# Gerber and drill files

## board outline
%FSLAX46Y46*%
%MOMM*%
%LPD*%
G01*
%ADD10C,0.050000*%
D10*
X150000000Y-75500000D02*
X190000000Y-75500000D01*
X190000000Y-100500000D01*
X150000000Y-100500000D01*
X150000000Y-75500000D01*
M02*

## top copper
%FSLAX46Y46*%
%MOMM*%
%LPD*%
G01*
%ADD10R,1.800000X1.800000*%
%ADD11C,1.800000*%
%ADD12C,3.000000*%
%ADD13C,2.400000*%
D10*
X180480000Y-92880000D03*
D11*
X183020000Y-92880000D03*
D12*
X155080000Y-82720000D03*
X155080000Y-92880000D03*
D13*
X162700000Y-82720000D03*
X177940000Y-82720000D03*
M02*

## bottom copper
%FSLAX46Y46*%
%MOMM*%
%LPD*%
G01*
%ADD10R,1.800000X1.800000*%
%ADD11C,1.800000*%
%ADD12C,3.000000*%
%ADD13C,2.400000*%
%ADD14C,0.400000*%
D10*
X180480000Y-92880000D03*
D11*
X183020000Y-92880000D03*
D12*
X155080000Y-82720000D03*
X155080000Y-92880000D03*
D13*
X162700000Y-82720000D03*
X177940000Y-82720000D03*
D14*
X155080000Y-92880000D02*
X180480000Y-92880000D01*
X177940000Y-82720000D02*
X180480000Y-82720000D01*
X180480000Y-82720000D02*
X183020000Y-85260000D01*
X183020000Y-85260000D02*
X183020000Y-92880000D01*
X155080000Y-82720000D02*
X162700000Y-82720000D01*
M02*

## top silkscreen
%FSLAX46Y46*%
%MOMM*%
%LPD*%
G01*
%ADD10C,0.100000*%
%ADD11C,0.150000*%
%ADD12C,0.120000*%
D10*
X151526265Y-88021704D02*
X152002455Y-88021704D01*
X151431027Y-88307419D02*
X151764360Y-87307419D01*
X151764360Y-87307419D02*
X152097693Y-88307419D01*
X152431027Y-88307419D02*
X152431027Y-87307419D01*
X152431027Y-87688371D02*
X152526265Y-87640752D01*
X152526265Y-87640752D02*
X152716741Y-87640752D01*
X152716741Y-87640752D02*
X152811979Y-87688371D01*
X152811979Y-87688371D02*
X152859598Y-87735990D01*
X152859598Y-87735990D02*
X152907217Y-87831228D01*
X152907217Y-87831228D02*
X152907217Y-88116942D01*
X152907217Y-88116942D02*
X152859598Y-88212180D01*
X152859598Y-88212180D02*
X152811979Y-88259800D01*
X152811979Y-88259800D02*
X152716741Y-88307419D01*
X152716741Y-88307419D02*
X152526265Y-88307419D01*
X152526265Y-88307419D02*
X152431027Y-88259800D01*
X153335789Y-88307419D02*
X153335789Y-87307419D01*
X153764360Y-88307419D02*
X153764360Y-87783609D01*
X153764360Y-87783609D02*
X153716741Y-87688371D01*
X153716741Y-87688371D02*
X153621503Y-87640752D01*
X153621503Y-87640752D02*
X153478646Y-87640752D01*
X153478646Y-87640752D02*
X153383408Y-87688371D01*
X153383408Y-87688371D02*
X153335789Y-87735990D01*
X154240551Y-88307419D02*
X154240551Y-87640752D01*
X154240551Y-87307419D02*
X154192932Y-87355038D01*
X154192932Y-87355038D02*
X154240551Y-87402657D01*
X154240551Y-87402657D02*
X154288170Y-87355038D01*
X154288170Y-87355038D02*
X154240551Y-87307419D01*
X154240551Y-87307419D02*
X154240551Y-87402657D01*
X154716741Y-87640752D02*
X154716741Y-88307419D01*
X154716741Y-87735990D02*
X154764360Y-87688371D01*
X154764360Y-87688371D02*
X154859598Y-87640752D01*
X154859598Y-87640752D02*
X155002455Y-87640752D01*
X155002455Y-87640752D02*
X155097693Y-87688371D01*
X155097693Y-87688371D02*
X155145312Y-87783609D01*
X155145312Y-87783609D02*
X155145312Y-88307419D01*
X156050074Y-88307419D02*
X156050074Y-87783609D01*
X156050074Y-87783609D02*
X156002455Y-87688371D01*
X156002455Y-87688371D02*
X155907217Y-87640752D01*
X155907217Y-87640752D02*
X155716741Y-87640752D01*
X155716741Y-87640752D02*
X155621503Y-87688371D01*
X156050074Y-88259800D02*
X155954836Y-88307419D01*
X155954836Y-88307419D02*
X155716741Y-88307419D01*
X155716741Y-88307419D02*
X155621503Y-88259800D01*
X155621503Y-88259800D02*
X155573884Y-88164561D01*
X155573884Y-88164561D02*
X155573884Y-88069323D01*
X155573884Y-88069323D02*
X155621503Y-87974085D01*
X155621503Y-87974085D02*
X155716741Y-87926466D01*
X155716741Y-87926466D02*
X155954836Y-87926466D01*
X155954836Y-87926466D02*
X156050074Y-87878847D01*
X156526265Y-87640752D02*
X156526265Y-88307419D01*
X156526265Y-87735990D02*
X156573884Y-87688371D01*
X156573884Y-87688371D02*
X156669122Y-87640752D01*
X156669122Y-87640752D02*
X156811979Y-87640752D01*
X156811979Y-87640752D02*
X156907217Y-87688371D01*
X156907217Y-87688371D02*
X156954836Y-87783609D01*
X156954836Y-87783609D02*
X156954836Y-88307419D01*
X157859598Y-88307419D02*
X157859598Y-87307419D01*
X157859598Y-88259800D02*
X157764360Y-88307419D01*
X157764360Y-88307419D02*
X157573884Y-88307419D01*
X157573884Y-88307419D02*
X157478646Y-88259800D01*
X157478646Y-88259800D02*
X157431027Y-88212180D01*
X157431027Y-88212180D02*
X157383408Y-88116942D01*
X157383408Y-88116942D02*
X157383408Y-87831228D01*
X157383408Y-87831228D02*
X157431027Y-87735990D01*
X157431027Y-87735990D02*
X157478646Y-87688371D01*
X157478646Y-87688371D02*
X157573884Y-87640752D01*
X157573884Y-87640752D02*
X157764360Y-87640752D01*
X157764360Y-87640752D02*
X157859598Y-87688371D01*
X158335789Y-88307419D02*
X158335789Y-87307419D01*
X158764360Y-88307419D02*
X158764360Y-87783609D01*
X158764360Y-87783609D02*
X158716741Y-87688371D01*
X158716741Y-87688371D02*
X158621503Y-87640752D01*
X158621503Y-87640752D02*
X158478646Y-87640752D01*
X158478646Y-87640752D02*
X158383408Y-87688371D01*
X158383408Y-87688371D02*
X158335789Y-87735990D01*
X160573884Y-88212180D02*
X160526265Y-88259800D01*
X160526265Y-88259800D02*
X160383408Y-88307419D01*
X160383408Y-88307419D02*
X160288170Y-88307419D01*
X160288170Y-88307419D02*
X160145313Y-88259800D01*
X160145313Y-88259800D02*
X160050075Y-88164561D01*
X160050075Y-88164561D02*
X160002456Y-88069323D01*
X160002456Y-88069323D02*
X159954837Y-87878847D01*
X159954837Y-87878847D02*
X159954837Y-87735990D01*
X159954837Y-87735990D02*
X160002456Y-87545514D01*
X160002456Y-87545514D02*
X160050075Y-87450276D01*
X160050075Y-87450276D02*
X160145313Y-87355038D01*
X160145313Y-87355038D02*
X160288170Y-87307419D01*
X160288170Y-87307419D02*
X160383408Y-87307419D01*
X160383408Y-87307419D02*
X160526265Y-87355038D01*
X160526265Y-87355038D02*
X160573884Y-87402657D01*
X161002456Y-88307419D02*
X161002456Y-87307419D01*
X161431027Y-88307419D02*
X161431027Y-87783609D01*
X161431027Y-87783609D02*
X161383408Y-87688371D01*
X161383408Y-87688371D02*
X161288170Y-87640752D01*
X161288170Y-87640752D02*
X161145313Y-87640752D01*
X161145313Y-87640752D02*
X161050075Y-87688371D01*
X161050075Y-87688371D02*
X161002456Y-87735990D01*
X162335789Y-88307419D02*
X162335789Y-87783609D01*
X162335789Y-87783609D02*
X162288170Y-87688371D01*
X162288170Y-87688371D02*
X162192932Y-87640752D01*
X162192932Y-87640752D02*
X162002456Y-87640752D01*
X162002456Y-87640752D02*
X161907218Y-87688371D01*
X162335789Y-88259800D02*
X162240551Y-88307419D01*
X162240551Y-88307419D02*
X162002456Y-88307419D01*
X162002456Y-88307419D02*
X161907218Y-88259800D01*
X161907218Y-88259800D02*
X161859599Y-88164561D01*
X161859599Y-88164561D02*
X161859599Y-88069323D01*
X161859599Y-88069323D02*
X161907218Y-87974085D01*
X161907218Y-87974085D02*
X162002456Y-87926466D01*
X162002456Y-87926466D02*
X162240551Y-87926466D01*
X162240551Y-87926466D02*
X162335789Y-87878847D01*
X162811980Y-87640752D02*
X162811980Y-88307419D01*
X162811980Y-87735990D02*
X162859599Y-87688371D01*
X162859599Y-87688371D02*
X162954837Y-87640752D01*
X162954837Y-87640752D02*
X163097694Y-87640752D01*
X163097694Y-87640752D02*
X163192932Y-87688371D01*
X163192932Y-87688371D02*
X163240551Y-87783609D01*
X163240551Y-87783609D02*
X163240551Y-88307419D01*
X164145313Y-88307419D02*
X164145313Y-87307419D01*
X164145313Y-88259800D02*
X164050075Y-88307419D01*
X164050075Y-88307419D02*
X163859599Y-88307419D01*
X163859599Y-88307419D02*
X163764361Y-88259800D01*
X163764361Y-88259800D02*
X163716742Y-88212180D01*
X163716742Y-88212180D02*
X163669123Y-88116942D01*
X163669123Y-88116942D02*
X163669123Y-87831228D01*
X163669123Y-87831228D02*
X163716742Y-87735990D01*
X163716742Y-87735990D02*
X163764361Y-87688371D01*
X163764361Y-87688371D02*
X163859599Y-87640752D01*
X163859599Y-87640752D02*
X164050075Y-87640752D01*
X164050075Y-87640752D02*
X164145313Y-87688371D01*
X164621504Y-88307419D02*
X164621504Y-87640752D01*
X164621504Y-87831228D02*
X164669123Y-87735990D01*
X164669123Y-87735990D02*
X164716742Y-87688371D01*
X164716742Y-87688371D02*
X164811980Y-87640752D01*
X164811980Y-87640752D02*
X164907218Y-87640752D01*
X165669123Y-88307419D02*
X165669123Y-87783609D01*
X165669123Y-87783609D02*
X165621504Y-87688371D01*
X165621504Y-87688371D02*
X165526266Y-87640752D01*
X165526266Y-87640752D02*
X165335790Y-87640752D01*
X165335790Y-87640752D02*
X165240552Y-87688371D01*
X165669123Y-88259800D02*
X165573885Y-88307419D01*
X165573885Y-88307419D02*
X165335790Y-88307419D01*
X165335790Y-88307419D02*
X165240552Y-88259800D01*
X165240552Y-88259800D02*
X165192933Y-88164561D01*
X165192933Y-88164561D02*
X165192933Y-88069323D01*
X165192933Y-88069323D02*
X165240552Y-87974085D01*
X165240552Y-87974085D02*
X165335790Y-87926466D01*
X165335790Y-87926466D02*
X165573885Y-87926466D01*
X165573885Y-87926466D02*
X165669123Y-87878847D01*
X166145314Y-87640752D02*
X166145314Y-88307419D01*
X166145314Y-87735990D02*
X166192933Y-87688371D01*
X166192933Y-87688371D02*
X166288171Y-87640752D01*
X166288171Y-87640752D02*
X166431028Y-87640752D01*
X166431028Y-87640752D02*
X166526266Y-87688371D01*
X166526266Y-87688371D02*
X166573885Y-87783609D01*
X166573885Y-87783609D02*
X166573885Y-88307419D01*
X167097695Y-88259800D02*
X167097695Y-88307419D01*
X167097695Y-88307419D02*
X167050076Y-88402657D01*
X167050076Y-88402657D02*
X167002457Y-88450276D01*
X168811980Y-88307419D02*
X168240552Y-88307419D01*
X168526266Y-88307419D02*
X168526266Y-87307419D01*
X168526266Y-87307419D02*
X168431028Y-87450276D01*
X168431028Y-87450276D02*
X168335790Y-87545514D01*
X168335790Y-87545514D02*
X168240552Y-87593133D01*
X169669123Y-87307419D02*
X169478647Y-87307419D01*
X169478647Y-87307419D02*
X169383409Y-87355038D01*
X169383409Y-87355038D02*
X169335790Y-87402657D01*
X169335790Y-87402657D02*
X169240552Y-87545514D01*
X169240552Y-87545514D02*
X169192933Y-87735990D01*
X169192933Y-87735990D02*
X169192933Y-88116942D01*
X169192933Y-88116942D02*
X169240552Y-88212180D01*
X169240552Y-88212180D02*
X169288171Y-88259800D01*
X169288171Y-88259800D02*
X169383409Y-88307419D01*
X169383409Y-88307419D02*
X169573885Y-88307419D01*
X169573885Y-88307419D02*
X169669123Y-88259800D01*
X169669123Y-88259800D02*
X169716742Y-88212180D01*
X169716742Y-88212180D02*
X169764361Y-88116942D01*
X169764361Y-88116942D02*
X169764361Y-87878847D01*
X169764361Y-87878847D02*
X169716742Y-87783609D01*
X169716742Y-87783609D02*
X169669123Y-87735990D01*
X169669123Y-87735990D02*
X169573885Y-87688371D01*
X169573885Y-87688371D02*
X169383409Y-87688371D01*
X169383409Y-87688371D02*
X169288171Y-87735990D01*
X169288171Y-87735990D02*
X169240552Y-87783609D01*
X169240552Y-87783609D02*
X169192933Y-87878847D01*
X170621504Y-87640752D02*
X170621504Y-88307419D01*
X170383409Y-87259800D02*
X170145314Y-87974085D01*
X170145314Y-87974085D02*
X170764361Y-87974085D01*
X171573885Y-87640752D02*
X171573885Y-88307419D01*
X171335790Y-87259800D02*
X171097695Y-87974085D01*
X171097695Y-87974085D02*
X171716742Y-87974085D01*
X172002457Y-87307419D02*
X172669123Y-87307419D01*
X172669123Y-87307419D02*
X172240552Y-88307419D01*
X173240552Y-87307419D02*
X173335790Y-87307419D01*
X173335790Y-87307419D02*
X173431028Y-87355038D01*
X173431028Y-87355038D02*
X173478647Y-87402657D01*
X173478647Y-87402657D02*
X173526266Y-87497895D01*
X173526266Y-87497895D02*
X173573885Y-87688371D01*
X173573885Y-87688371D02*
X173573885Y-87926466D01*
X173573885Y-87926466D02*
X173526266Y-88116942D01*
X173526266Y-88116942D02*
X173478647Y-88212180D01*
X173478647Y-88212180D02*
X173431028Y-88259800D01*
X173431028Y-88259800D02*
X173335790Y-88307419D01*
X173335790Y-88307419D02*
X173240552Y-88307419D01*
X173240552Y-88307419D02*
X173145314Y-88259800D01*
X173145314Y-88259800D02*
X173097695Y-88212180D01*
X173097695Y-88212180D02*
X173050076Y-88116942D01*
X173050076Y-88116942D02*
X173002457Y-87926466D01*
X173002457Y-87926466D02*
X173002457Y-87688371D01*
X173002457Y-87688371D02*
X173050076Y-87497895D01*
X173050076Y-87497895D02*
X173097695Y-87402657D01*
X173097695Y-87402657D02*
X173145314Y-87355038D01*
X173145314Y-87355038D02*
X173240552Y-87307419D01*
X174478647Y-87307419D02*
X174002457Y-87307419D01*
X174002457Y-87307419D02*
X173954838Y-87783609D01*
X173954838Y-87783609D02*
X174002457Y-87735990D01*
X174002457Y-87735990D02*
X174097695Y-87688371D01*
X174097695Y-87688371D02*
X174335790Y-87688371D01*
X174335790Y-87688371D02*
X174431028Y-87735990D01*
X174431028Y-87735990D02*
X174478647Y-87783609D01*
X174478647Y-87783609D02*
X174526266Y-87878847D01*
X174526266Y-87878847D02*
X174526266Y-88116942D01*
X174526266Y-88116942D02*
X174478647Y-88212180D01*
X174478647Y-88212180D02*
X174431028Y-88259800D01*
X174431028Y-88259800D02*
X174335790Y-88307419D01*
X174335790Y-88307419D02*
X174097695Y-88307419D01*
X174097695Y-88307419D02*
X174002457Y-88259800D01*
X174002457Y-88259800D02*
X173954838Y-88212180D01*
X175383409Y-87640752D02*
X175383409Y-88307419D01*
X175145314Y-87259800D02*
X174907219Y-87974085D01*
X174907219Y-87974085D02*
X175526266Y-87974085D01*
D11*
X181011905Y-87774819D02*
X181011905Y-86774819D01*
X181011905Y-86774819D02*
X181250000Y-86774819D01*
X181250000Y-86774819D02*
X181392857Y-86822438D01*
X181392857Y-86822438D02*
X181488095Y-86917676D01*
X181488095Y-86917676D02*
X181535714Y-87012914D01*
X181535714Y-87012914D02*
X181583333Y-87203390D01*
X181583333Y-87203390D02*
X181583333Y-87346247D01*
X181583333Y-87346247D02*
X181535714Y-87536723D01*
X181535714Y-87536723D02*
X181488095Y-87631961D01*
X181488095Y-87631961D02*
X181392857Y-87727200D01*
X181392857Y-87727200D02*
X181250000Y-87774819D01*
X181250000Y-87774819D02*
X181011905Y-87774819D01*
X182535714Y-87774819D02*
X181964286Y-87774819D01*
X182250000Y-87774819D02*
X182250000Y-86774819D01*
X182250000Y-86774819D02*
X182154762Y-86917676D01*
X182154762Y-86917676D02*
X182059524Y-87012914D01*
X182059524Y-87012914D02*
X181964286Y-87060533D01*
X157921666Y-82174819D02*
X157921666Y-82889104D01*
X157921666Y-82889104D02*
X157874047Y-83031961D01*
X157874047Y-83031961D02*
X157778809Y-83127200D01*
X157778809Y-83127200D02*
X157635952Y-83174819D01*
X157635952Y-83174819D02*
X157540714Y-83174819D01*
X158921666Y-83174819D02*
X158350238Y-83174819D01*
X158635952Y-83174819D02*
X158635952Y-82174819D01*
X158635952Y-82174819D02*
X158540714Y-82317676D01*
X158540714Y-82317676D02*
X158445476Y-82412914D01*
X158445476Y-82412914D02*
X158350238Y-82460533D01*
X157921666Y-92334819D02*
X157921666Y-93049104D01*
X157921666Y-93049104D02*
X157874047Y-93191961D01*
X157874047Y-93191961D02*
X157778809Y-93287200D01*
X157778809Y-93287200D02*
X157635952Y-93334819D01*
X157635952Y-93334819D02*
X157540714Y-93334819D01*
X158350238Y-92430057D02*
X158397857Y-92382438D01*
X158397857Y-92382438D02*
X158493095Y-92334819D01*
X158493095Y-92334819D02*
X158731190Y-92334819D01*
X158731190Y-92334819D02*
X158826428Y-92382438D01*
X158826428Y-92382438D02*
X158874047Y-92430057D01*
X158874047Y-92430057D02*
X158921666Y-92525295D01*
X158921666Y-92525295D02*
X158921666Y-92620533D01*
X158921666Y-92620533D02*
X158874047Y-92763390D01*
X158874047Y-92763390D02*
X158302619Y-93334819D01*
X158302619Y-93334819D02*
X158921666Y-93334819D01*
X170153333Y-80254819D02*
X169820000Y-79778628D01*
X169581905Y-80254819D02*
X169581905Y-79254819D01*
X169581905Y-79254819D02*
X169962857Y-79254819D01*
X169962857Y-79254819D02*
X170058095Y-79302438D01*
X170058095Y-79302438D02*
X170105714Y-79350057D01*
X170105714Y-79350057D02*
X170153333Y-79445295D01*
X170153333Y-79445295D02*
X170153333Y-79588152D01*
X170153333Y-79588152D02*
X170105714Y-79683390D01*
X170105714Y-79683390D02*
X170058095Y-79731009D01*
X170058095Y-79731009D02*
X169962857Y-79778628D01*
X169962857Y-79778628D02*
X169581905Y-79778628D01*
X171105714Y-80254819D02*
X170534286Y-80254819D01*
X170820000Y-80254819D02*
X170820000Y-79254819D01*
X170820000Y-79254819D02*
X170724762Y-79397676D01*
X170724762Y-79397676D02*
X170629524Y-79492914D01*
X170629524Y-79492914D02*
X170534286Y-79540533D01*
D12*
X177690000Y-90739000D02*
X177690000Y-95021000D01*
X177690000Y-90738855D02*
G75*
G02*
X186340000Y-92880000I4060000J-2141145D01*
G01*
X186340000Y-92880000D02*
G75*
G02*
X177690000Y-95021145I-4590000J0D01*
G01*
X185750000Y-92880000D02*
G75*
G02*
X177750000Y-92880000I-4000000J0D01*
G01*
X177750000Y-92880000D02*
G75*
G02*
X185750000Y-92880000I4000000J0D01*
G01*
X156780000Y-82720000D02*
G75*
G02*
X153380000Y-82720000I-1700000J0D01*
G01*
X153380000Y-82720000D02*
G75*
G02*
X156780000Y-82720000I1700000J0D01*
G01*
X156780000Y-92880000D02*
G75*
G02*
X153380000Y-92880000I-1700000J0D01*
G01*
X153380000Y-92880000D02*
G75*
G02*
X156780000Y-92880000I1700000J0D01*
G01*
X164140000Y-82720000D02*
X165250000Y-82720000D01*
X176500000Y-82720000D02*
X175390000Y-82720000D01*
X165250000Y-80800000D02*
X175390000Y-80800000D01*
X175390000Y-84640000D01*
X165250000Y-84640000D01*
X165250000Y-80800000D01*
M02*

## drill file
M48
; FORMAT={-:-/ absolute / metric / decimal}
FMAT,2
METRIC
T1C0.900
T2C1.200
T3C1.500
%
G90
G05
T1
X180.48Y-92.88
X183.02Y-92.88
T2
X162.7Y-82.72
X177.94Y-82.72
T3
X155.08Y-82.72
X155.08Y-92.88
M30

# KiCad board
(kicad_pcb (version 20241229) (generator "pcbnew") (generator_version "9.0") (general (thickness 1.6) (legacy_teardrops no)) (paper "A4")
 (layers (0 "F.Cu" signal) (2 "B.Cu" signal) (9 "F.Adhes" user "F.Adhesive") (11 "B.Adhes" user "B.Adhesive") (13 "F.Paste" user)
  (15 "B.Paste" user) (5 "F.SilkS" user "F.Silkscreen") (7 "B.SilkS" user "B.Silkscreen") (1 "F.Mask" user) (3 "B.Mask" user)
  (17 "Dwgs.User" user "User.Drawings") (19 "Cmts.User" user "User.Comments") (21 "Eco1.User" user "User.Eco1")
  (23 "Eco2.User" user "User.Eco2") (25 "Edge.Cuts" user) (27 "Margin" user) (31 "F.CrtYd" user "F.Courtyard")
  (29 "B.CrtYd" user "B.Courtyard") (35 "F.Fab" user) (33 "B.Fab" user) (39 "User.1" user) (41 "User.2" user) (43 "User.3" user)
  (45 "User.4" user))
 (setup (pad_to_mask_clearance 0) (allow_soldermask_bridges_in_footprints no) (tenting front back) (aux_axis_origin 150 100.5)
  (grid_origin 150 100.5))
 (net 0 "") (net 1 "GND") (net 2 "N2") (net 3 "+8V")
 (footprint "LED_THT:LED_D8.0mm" (layer "F.Cu") (at 180.48 92.88)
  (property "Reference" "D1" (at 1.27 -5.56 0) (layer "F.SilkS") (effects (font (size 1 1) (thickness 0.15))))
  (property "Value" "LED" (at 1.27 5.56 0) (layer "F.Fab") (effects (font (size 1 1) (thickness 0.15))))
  (fp_line (start -2.79 -2.141) (end -2.79 2.141) (stroke (width 0.12) (type solid)) (layer "F.SilkS"))
  (fp_arc (start -2.79 -2.141145) (mid 2.372883 -4.45553) (end 5.86 0) (stroke (width 0.12) (type solid)) (layer "F.SilkS"))
  (fp_arc (start 5.86 0) (mid 2.372883 4.45553) (end -2.79 2.141145) (stroke (width 0.12) (type solid)) (layer "F.SilkS"))
  (fp_circle (center 1.27 0) (end 5.27 0) (stroke (width 0.12) (type solid)) (fill no) (layer "F.SilkS"))
  (pad "1" thru_hole rect (at 0 0) (size 1.8 1.8) (drill 0.9) (layers "*.Cu" "*.Mask") (remove_unused_layers no) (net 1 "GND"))
  (pad "2" thru_hole circle (at 2.54 0) (size 1.8 1.8) (drill 0.9) (layers "*.Cu" "*.Mask") (remove_unused_layers no) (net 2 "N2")))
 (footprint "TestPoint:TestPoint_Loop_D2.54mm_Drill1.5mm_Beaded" (layer "F.Cu") (at 155.08 82.72)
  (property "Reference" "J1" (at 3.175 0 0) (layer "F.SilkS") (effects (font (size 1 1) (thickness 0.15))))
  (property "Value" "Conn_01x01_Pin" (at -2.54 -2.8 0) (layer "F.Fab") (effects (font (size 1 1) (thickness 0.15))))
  (fp_circle (center 0 0) (end 1.7 0) (stroke (width 0.12) (type solid)) (fill no) (layer "F.SilkS"))
  (pad "1" thru_hole circle (at 0 0) (size 3 3) (drill 1.5) (layers "*.Cu" "*.Mask") (remove_unused_layers no) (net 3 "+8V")))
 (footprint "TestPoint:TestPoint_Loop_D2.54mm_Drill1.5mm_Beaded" (layer "F.Cu") (at 155.08 92.88)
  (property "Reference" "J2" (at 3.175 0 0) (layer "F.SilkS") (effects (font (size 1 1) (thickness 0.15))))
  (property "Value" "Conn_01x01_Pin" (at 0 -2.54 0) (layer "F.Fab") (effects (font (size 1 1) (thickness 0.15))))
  (fp_circle (center 0 0) (end 1.7 0) (stroke (width 0.12) (type solid)) (fill no) (layer "F.SilkS"))
  (pad "1" thru_hole circle (at 0 0) (size 3 3) (drill 1.5) (layers "*.Cu" "*.Mask") (remove_unused_layers no) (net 1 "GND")))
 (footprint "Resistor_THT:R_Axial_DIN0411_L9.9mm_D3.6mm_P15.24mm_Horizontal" (layer "F.Cu") (at 162.7 82.72)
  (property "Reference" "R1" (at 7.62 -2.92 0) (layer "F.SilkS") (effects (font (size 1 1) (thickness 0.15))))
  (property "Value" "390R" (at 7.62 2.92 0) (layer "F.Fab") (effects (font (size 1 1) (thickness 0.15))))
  (fp_line (start 1.44 0) (end 2.55 0) (stroke (width 0.12) (type solid)) (layer "F.SilkS"))
  (fp_line (start 13.8 0) (end 12.69 0) (stroke (width 0.12) (type solid)) (layer "F.SilkS"))
  (fp_rect (start 2.55 -1.92) (end 12.69 1.92) (stroke (width 0.12) (type solid)) (fill no) (layer "F.SilkS"))
  (pad "1" thru_hole circle (at 0 0) (size 2.4 2.4) (drill 1.2) (layers "*.Cu" "*.Mask") (remove_unused_layers no) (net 3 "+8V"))
  (pad "2" thru_hole circle (at 15.24 0) (size 2.4 2.4) (drill 1.2) (layers "*.Cu" "*.Mask") (remove_unused_layers no) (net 2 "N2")))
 (gr_rect (start 150 75.5) (end 190 100.5) (stroke (width 0.05) (type solid)) (fill no) (layer "Edge.Cuts"))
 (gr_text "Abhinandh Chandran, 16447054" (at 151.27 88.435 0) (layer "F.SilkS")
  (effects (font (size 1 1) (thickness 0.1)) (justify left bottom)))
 (segment (start 155.08 92.88) (end 180.48 92.88) (width 0.4) (layer "B.Cu") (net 1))
 (segment (start 177.94 82.72) (end 180.48 82.72) (width 0.4) (layer "B.Cu") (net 2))
 (segment (start 180.48 82.72) (end 183.02 85.26) (width 0.4) (layer "B.Cu") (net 2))
 (segment (start 183.02 85.26) (end 183.02 92.88) (width 0.4) (layer "B.Cu") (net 2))
 (segment (start 155.08 82.72) (end 162.7 82.72) (width 0.4) (layer "B.Cu") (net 3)))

